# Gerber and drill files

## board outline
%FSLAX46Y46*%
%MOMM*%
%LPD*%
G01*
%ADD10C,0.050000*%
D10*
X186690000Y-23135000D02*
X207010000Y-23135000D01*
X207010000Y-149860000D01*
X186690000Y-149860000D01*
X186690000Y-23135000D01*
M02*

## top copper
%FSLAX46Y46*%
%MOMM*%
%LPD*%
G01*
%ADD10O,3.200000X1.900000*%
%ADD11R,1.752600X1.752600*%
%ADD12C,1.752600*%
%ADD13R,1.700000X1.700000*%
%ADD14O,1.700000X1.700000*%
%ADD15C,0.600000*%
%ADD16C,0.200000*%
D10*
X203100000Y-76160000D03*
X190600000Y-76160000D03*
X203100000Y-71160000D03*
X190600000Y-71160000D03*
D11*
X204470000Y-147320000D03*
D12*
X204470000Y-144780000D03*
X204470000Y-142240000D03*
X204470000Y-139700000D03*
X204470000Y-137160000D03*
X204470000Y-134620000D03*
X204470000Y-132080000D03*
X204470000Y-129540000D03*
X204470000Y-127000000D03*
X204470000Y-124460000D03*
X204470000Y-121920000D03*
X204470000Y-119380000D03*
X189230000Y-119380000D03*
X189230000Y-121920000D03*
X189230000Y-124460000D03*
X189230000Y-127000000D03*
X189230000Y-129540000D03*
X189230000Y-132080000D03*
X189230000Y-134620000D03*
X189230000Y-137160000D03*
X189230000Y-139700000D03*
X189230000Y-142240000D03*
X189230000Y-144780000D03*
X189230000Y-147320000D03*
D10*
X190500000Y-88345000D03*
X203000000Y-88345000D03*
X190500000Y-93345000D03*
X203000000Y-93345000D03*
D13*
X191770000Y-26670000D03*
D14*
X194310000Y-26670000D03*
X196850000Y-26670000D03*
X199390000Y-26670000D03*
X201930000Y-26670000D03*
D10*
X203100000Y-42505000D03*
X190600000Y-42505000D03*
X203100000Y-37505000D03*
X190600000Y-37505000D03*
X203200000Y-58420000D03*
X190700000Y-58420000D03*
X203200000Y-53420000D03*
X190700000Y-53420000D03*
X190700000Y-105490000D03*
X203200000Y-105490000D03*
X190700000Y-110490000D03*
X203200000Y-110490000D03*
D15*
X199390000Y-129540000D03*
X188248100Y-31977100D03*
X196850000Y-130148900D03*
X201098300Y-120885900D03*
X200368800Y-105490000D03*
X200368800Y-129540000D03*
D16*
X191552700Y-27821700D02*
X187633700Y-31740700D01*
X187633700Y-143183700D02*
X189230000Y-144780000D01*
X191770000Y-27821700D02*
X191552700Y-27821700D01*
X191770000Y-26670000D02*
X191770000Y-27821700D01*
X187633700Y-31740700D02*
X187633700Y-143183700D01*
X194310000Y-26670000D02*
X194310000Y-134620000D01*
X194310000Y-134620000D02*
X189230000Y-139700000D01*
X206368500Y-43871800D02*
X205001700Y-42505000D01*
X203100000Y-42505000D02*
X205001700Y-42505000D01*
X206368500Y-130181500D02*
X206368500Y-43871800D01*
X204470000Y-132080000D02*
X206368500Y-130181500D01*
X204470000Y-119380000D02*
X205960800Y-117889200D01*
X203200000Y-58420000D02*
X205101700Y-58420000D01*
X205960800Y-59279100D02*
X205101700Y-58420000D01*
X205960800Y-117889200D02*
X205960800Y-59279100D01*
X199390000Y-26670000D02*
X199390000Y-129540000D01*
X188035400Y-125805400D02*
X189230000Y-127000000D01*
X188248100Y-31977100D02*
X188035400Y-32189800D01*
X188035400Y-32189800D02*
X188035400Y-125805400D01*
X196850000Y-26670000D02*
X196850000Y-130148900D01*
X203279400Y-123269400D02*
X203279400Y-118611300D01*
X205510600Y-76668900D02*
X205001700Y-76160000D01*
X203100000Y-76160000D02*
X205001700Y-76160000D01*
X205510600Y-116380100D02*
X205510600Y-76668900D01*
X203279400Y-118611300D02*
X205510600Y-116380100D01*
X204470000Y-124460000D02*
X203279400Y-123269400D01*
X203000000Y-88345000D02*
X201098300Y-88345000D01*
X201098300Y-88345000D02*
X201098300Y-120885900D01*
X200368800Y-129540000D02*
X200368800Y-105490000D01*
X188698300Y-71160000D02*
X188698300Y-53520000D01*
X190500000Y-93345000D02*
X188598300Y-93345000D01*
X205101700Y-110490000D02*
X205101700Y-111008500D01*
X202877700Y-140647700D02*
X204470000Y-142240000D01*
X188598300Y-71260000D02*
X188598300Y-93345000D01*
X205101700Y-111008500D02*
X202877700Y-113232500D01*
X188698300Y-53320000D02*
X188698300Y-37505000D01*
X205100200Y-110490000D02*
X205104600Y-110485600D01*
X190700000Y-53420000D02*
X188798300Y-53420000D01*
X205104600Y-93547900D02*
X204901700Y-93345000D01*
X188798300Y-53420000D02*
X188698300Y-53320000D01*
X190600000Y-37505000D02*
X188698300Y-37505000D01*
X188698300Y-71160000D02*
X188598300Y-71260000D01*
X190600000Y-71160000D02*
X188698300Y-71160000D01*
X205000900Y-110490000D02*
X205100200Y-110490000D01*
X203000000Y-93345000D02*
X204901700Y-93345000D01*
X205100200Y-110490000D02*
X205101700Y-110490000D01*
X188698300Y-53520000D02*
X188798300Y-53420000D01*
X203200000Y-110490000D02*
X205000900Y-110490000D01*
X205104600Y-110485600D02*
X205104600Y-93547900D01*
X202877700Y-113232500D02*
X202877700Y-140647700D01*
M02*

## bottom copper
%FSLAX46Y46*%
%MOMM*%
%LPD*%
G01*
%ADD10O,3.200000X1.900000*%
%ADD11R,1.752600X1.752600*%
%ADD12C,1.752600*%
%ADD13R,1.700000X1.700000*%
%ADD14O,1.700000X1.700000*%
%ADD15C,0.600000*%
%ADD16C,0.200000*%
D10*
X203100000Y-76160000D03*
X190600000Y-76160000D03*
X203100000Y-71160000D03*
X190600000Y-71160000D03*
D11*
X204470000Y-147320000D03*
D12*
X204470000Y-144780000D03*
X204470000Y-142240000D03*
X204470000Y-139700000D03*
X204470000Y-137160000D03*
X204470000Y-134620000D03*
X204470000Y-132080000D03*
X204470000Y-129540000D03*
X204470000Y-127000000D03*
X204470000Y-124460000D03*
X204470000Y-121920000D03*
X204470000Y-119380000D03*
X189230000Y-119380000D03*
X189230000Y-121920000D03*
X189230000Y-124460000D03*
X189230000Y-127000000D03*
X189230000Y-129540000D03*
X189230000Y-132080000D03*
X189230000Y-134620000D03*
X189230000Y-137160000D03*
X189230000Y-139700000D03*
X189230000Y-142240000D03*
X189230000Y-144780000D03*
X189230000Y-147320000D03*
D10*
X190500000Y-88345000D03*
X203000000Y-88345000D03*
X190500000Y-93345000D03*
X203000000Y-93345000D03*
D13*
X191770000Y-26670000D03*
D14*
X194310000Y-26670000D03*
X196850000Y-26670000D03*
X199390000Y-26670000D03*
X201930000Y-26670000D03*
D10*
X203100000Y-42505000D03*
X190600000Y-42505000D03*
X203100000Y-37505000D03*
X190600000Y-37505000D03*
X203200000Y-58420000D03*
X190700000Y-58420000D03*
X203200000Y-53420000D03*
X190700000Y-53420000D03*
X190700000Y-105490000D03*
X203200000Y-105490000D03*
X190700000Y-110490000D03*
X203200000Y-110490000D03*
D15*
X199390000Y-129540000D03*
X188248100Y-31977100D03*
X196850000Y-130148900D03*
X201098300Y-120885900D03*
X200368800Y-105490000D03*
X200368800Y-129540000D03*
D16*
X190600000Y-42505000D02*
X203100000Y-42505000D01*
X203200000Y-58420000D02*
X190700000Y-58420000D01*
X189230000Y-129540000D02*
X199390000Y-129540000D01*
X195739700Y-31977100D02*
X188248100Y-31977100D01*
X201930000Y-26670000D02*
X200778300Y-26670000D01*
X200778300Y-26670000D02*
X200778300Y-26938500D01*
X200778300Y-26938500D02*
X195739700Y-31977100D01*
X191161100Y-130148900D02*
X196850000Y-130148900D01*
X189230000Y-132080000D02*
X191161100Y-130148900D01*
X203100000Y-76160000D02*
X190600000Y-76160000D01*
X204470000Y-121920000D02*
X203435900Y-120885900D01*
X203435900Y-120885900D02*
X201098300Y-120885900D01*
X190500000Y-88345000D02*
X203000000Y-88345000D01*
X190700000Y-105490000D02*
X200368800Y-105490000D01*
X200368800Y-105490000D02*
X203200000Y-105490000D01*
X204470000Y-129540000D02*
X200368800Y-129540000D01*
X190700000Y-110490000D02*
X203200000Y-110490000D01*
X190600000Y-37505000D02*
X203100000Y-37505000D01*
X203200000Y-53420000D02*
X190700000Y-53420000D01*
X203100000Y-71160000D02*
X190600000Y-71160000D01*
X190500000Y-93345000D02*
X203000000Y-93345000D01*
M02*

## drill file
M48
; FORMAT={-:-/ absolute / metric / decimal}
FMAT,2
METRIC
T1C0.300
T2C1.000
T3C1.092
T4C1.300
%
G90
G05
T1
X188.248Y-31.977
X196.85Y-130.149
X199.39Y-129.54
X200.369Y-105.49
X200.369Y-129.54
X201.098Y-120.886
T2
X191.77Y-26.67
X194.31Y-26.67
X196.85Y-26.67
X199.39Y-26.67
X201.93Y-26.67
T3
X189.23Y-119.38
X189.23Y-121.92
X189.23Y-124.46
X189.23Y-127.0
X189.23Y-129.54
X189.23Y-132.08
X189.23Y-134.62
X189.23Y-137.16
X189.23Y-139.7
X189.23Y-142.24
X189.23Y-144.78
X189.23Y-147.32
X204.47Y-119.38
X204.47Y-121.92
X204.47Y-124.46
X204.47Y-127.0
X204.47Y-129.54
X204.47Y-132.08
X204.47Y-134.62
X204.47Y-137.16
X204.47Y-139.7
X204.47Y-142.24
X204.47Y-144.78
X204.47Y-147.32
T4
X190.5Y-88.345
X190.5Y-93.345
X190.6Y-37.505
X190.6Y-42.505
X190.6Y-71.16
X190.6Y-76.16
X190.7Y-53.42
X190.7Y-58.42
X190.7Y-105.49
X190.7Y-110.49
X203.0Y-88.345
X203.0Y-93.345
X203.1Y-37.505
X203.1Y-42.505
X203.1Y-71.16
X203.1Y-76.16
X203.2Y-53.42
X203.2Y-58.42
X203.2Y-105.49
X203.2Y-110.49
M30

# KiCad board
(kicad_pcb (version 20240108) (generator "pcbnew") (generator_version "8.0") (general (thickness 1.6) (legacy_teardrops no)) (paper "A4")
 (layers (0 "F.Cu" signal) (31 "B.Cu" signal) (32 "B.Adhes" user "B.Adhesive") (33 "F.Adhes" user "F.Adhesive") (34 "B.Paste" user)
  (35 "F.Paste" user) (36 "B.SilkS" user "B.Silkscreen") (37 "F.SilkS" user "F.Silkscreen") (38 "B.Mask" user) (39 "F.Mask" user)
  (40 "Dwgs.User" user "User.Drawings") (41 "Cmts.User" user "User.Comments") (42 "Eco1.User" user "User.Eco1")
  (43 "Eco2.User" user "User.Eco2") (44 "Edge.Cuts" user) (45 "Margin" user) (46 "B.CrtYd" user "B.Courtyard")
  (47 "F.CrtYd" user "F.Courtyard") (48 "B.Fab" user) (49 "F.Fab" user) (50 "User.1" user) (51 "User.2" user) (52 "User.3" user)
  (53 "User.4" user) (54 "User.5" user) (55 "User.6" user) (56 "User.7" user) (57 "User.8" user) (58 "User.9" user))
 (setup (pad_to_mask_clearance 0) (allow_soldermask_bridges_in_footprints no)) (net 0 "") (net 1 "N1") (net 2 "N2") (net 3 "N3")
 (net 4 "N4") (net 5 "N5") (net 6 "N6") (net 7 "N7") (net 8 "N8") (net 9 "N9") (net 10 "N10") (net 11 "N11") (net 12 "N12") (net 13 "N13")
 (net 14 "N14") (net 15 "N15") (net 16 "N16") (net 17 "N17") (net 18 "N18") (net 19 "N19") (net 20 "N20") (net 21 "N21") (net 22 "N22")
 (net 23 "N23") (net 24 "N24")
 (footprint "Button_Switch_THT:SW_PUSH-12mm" (layer "F.Cu") (at 203.1 76.16 180)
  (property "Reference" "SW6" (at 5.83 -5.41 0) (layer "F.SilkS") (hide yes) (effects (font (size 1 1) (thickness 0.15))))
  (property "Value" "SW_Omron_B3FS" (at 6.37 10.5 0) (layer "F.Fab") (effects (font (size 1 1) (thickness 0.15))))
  (pad "1" thru_hole oval (at 0 0 180) (size 3.2 1.9) (drill 1.3) (layers "*.Cu" "*.Mask") (remove_unused_layers no) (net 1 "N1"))
  (pad "1" thru_hole oval (at 12.5 0 180) (size 3.2 1.9) (drill 1.3) (layers "*.Cu" "*.Mask") (remove_unused_layers no) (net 1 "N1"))
  (pad "2" thru_hole oval (at 0 5 180) (size 3.2 1.9) (drill 1.3) (layers "*.Cu" "*.Mask") (remove_unused_layers no) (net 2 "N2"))
  (pad "2" thru_hole oval (at 12.5 5 180) (size 3.2 1.9) (drill 1.3) (layers "*.Cu" "*.Mask") (remove_unused_layers no) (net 2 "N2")))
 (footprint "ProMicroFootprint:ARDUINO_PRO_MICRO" (layer "F.Cu") (at 196.85 133.35 90)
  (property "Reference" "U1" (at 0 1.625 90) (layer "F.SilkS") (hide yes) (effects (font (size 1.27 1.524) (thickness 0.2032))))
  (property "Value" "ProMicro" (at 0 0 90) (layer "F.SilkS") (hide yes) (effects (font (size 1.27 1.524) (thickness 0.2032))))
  (pad "1" thru_hole rect (at -13.97 7.62 90) (size 1.7526 1.7526) (drill 1.0922) (layers "*.Cu" "*.SilkS" "*.Mask")
   (remove_unused_layers no) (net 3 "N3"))
  (pad "2" thru_hole circle (at -11.43 7.62 90) (size 1.7526 1.7526) (drill 1.0922) (layers "*.Cu" "*.SilkS" "*.Mask")
   (remove_unused_layers no) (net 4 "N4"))
  (pad "3" thru_hole circle (at -8.89 7.62 90) (size 1.7526 1.7526) (drill 1.0922) (layers "*.Cu" "*.SilkS" "*.Mask")
   (remove_unused_layers no) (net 2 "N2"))
  (pad "4" thru_hole circle (at -6.35 7.62 90) (size 1.7526 1.7526) (drill 1.0922) (layers "*.Cu" "*.SilkS" "*.Mask")
   (remove_unused_layers no) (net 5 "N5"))
  (pad "5" thru_hole circle (at -3.81 7.62 90) (size 1.7526 1.7526) (drill 1.0922) (layers "*.Cu" "*.SilkS" "*.Mask")
   (remove_unused_layers no) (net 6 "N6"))
  (pad "6" thru_hole circle (at -1.27 7.62 90) (size 1.7526 1.7526) (drill 1.0922) (layers "*.Cu" "*.SilkS" "*.Mask")
   (remove_unused_layers no) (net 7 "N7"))
  (pad "7" thru_hole circle (at 1.27 7.62 90) (size 1.7526 1.7526) (drill 1.0922) (layers "*.Cu" "*.SilkS" "*.Mask")
   (remove_unused_layers no) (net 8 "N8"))
  (pad "8" thru_hole circle (at 3.81 7.62 90) (size 1.7526 1.7526) (drill 1.0922) (layers "*.Cu" "*.SilkS" "*.Mask")
   (remove_unused_layers no) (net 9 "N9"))
  (pad "9" thru_hole circle (at 6.35 7.62 90) (size 1.7526 1.7526) (drill 1.0922) (layers "*.Cu" "*.SilkS" "*.Mask")
   (remove_unused_layers no) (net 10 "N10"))
  (pad "10" thru_hole circle (at 8.89 7.62 90) (size 1.7526 1.7526) (drill 1.0922) (layers "*.Cu" "*.SilkS" "*.Mask")
   (remove_unused_layers no) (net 1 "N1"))
  (pad "11" thru_hole circle (at 11.43 7.62 90) (size 1.7526 1.7526) (drill 1.0922) (layers "*.Cu" "*.SilkS" "*.Mask")
   (remove_unused_layers no) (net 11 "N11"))
  (pad "12" thru_hole circle (at 13.97 7.62 90) (size 1.7526 1.7526) (drill 1.0922) (layers "*.Cu" "*.SilkS" "*.Mask")
   (remove_unused_layers no) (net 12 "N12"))
  (pad "13" thru_hole circle (at 13.97 -7.62 90) (size 1.7526 1.7526) (drill 1.0922) (layers "*.Cu" "*.SilkS" "*.Mask")
   (remove_unused_layers no) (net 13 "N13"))
  (pad "14" thru_hole circle (at 11.43 -7.62 90) (size 1.7526 1.7526) (drill 1.0922) (layers "*.Cu" "*.SilkS" "*.Mask")
   (remove_unused_layers no) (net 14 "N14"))
  (pad "15" thru_hole circle (at 8.89 -7.62 90) (size 1.7526 1.7526) (drill 1.0922) (layers "*.Cu" "*.SilkS" "*.Mask")
   (remove_unused_layers no) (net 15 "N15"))
  (pad "16" thru_hole circle (at 6.35 -7.62 90) (size 1.7526 1.7526) (drill 1.0922) (layers "*.Cu" "*.SilkS" "*.Mask")
   (remove_unused_layers no) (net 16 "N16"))
  (pad "17" thru_hole circle (at 3.81 -7.62 90) (size 1.7526 1.7526) (drill 1.0922) (layers "*.Cu" "*.SilkS" "*.Mask")
   (remove_unused_layers no) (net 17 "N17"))
  (pad "18" thru_hole circle (at 1.27 -7.62 90) (size 1.7526 1.7526) (drill 1.0922) (layers "*.Cu" "*.SilkS" "*.Mask")
   (remove_unused_layers no) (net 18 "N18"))
  (pad "19" thru_hole circle (at -1.27 -7.62 90) (size 1.7526 1.7526) (drill 1.0922) (layers "*.Cu" "*.SilkS" "*.Mask")
   (remove_unused_layers no) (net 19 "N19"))
  (pad "20" thru_hole circle (at -3.81 -7.62 90) (size 1.7526 1.7526) (drill 1.0922) (layers "*.Cu" "*.SilkS" "*.Mask")
   (remove_unused_layers no) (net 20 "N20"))
  (pad "21" thru_hole circle (at -6.35 -7.62 90) (size 1.7526 1.7526) (drill 1.0922) (layers "*.Cu" "*.SilkS" "*.Mask")
   (remove_unused_layers no) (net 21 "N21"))
  (pad "22" thru_hole circle (at -8.89 -7.62 90) (size 1.7526 1.7526) (drill 1.0922) (layers "*.Cu" "*.SilkS" "*.Mask")
   (remove_unused_layers no) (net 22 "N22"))
  (pad "23" thru_hole circle (at -11.43 -7.62 90) (size 1.7526 1.7526) (drill 1.0922) (layers "*.Cu" "*.SilkS" "*.Mask")
   (remove_unused_layers no) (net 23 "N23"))
  (pad "24" thru_hole circle (at -13.97 -7.62 90) (size 1.7526 1.7526) (drill 1.0922) (layers "*.Cu" "*.SilkS" "*.Mask")
   (remove_unused_layers no) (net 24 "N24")))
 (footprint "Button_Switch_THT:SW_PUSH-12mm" (layer "F.Cu") (at 190.5 88.345)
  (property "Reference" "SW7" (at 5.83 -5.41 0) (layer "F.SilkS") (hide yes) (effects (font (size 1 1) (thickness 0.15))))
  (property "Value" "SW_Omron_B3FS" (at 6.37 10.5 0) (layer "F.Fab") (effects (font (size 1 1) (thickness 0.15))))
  (pad "1" thru_hole oval (at 0 0) (size 3.2 1.9) (drill 1.3) (layers "*.Cu" "*.Mask") (remove_unused_layers no) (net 11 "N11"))
  (pad "1" thru_hole oval (at 12.5 0) (size 3.2 1.9) (drill 1.3) (layers "*.Cu" "*.Mask") (remove_unused_layers no) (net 11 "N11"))
  (pad "2" thru_hole oval (at 0 5) (size 3.2 1.9) (drill 1.3) (layers "*.Cu" "*.Mask") (remove_unused_layers no) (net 2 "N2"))
  (pad "2" thru_hole oval (at 12.5 5) (size 3.2 1.9) (drill 1.3) (layers "*.Cu" "*.Mask") (remove_unused_layers no) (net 2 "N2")))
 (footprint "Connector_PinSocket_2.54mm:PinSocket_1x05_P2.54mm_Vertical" (layer "F.Cu") (at 191.77 26.67 90)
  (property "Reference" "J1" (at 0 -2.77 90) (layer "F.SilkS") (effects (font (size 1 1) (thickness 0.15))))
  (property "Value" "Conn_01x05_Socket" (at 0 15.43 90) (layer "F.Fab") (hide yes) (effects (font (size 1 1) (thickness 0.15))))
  (pad "1" thru_hole rect (at 0 0 90) (size 1.7 1.7) (drill 1) (layers "*.Cu" "*.Mask") (remove_unused_layers no) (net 23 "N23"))
  (pad "2" thru_hole oval (at 0 2.54 90) (size 1.7 1.7) (drill 1) (layers "*.Cu" "*.Mask") (remove_unused_layers no) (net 21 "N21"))
  (pad "3" thru_hole oval (at 0 5.08 90) (size 1.7 1.7) (drill 1) (layers "*.Cu" "*.Mask") (remove_unused_layers no) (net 18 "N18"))
  (pad "4" thru_hole oval (at 0 7.62 90) (size 1.7 1.7) (drill 1) (layers "*.Cu" "*.Mask") (remove_unused_layers no) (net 17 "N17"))
  (pad "5" thru_hole oval (at 0 10.16 90) (size 1.7 1.7) (drill 1) (layers "*.Cu" "*.Mask") (remove_unused_layers no) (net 16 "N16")))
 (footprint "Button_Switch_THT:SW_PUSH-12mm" (layer "F.Cu") (at 203.1 42.505 180)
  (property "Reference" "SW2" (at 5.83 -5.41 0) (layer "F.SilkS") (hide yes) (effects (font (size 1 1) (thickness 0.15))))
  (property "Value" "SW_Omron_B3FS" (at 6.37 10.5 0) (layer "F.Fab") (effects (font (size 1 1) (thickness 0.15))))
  (pad "1" thru_hole oval (at 0 0 180) (size 3.2 1.9) (drill 1.3) (layers "*.Cu" "*.Mask") (remove_unused_layers no) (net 8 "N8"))
  (pad "1" thru_hole oval (at 12.5 0 180) (size 3.2 1.9) (drill 1.3) (layers "*.Cu" "*.Mask") (remove_unused_layers no) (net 8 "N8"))
  (pad "2" thru_hole oval (at 0 5 180) (size 3.2 1.9) (drill 1.3) (layers "*.Cu" "*.Mask") (remove_unused_layers no) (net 2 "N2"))
  (pad "2" thru_hole oval (at 12.5 5 180) (size 3.2 1.9) (drill 1.3) (layers "*.Cu" "*.Mask") (remove_unused_layers no) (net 2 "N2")))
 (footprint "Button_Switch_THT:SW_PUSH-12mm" (layer "F.Cu") (at 203.2 58.42 180)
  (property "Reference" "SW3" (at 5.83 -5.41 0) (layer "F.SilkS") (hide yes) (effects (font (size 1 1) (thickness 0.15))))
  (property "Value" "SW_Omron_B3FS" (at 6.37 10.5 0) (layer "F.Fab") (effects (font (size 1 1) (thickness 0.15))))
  (pad "1" thru_hole oval (at 0 0 180) (size 3.2 1.9) (drill 1.3) (layers "*.Cu" "*.Mask") (remove_unused_layers no) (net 12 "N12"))
  (pad "1" thru_hole oval (at 12.5 0 180) (size 3.2 1.9) (drill 1.3) (layers "*.Cu" "*.Mask") (remove_unused_layers no) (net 12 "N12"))
  (pad "2" thru_hole oval (at 0 5 180) (size 3.2 1.9) (drill 1.3) (layers "*.Cu" "*.Mask") (remove_unused_layers no) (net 2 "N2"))
  (pad "2" thru_hole oval (at 12.5 5 180) (size 3.2 1.9) (drill 1.3) (layers "*.Cu" "*.Mask") (remove_unused_layers no) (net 2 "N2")))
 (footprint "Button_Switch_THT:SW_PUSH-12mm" (layer "F.Cu") (at 190.7 105.49)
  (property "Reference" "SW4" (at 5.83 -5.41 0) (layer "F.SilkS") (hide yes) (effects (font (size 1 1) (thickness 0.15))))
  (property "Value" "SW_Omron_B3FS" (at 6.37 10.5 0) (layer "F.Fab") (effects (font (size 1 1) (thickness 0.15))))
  (pad "1" thru_hole oval (at 0 0) (size 3.2 1.9) (drill 1.3) (layers "*.Cu" "*.Mask") (remove_unused_layers no) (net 9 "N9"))
  (pad "1" thru_hole oval (at 12.5 0) (size 3.2 1.9) (drill 1.3) (layers "*.Cu" "*.Mask") (remove_unused_layers no) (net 9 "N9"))
  (pad "2" thru_hole oval (at 0 5) (size 3.2 1.9) (drill 1.3) (layers "*.Cu" "*.Mask") (remove_unused_layers no) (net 2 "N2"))
  (pad "2" thru_hole oval (at 12.5 5) (size 3.2 1.9) (drill 1.3) (layers "*.Cu" "*.Mask") (remove_unused_layers no) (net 2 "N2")))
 (gr_rect (start 186.69 23.135) (end 207.01 149.86) (stroke (width 0.05) (type default)) (fill none) (layer "Edge.Cuts"))
 (segment (start 191.5527 27.8217) (end 187.6337 31.7407) (width 0.2) (layer "F.Cu") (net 23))
 (segment (start 187.6337 143.1837) (end 189.23 144.78) (width 0.2) (layer "F.Cu") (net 23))
 (segment (start 191.77 27.8217) (end 191.5527 27.8217) (width 0.2) (layer "F.Cu") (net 23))
 (segment (start 191.77 26.67) (end 191.77 27.8217) (width 0.2) (layer "F.Cu") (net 23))
 (segment (start 187.6337 31.7407) (end 187.6337 143.1837) (width 0.2) (layer "F.Cu") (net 23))
 (segment (start 194.31 26.67) (end 194.31 134.62) (width 0.2) (layer "F.Cu") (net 21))
 (segment (start 194.31 134.62) (end 189.23 139.7) (width 0.2) (layer "F.Cu") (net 21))
 (segment (start 206.3685 43.8718) (end 205.0017 42.505) (width 0.2) (layer "F.Cu") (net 8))
 (segment (start 203.1 42.505) (end 205.0017 42.505) (width 0.2) (layer "F.Cu") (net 8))
 (segment (start 206.3685 130.1815) (end 206.3685 43.8718) (width 0.2) (layer "F.Cu") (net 8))
 (segment (start 204.47 132.08) (end 206.3685 130.1815) (width 0.2) (layer "F.Cu") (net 8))
 (segment (start 190.6 42.505) (end 203.1 42.505) (width 0.2) (layer "B.Cu") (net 8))
 (segment (start 204.47 119.38) (end 205.9608 117.8892) (width 0.2) (layer "F.Cu") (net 12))
 (segment (start 203.2 58.42) (end 205.1017 58.42) (width 0.2) (layer "F.Cu") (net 12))
 (segment (start 205.9608 59.2791) (end 205.1017 58.42) (width 0.2) (layer "F.Cu") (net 12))
 (segment (start 205.9608 117.8892) (end 205.9608 59.2791) (width 0.2) (layer "F.Cu") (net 12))
 (segment (start 203.2 58.42) (end 190.7 58.42) (width 0.2) (layer "B.Cu") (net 12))
 (segment (start 199.39 26.67) (end 199.39 129.54) (width 0.2) (layer "F.Cu") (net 17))
 (via (at 199.39 129.54) (size 0.6) (drill 0.3) (layers "F.Cu" "B.Cu") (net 17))
 (segment (start 189.23 129.54) (end 199.39 129.54) (width 0.2) (layer "B.Cu") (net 17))
 (segment (start 188.0354 125.8054) (end 189.23 127) (width 0.2) (layer "F.Cu") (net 16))
 (segment (start 188.2481 31.9771) (end 188.0354 32.1898) (width 0.2) (layer "F.Cu") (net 16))
 (segment (start 188.0354 32.1898) (end 188.0354 125.8054) (width 0.2) (layer "F.Cu") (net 16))
 (via (at 188.2481 31.9771) (size 0.6) (drill 0.3) (layers "F.Cu" "B.Cu") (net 16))
 (segment (start 195.7397 31.9771) (end 188.2481 31.9771) (width 0.2) (layer "B.Cu") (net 16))
 (segment (start 201.93 26.67) (end 200.7783 26.67) (width 0.2) (layer "B.Cu") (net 16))
 (segment (start 200.7783 26.67) (end 200.7783 26.9385) (width 0.2) (layer "B.Cu") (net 16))
 (segment (start 200.7783 26.9385) (end 195.7397 31.9771) (width 0.2) (layer "B.Cu") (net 16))
 (segment (start 196.85 26.67) (end 196.85 130.1489) (width 0.2) (layer "F.Cu") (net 18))
 (via (at 196.85 130.1489) (size 0.6) (drill 0.3) (layers "F.Cu" "B.Cu") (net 18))
 (segment (start 191.1611 130.1489) (end 196.85 130.1489) (width 0.2) (layer "B.Cu") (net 18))
 (segment (start 189.23 132.08) (end 191.1611 130.1489) (width 0.2) (layer "B.Cu") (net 18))
 (segment (start 203.2794 123.2694) (end 203.2794 118.6113) (width 0.2) (layer "F.Cu") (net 1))
 (segment (start 205.5106 76.6689) (end 205.0017 76.16) (width 0.2) (layer "F.Cu") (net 1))
 (segment (start 203.1 76.16) (end 205.0017 76.16) (width 0.2) (layer "F.Cu") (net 1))
 (segment (start 205.5106 116.3801) (end 205.5106 76.6689) (width 0.2) (layer "F.Cu") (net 1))
 (segment (start 203.2794 118.6113) (end 205.5106 116.3801) (width 0.2) (layer "F.Cu") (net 1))
 (segment (start 204.47 124.46) (end 203.2794 123.2694) (width 0.2) (layer "F.Cu") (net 1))
 (segment (start 203.1 76.16) (end 190.6 76.16) (width 0.2) (layer "B.Cu") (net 1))
 (segment (start 203 88.345) (end 201.0983 88.345) (width 0.2) (layer "F.Cu") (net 11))
 (segment (start 201.0983 88.345) (end 201.0983 120.8859) (width 0.2) (layer "F.Cu") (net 11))
 (via (at 201.0983 120.8859) (size 0.6) (drill 0.3) (layers "F.Cu" "B.Cu") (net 11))
 (segment (start 204.47 121.92) (end 203.4359 120.8859) (width 0.2) (layer "B.Cu") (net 11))
 (segment (start 203.4359 120.8859) (end 201.0983 120.8859) (width 0.2) (layer "B.Cu") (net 11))
 (segment (start 190.5 88.345) (end 203 88.345) (width 0.2) (layer "B.Cu") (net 11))
 (segment (start 200.3688 129.54) (end 200.3688 105.49) (width 0.2) (layer "F.Cu") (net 9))
 (via (at 200.3688 105.49) (size 0.6) (drill 0.3) (layers "F.Cu" "B.Cu") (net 9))
 (via (at 200.3688 129.54) (size 0.6) (drill 0.3) (layers "F.Cu" "B.Cu") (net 9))
 (segment (start 190.7 105.49) (end 200.3688 105.49) (width 0.2) (layer "B.Cu") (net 9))
 (segment (start 200.3688 105.49) (end 203.2 105.49) (width 0.2) (layer "B.Cu") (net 9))
 (segment (start 204.47 129.54) (end 200.3688 129.54) (width 0.2) (layer "B.Cu") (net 9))
 (segment (start 188.6983 71.16) (end 188.6983 53.52) (width 0.2) (layer "F.Cu") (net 2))
 (segment (start 190.5 93.345) (end 188.5983 93.345) (width 0.2) (layer "F.Cu") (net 2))
 (segment (start 205.1017 110.49) (end 205.1017 111.0085) (width 0.2) (layer "F.Cu") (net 2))
 (segment (start 202.8777 140.6477) (end 204.47 142.24) (width 0.2) (layer "F.Cu") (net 2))
 (segment (start 188.5983 71.26) (end 188.5983 93.345) (width 0.2) (layer "F.Cu") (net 2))
 (segment (start 205.1017 111.0085) (end 202.8777 113.2325) (width 0.2) (layer "F.Cu") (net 2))
 (segment (start 188.6983 53.32) (end 188.6983 37.505) (width 0.2) (layer "F.Cu") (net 2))
 (segment (start 205.1002 110.49) (end 205.1046 110.4856) (width 0.2) (layer "F.Cu") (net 2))
 (segment (start 190.7 53.42) (end 188.7983 53.42) (width 0.2) (layer "F.Cu") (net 2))
 (segment (start 205.1046 93.5479) (end 204.9017 93.345) (width 0.2) (layer "F.Cu") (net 2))
 (segment (start 188.7983 53.42) (end 188.6983 53.32) (width 0.2) (layer "F.Cu") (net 2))
 (segment (start 190.6 37.505) (end 188.6983 37.505) (width 0.2) (layer "F.Cu") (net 2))
 (segment (start 188.6983 71.16) (end 188.5983 71.26) (width 0.2) (layer "F.Cu") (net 2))
 (segment (start 190.6 71.16) (end 188.6983 71.16) (width 0.2) (layer "F.Cu") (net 2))
 (segment (start 205.0009 110.49) (end 205.1002 110.49) (width 0.2) (layer "F.Cu") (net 2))
 (segment (start 203 93.345) (end 204.9017 93.345) (width 0.2) (layer "F.Cu") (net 2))
 (segment (start 205.1002 110.49) (end 205.1017 110.49) (width 0.2) (layer "F.Cu") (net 2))
 (segment (start 188.6983 53.52) (end 188.7983 53.42) (width 0.2) (layer "F.Cu") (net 2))
 (segment (start 203.2 110.49) (end 205.0009 110.49) (width 0.2) (layer "F.Cu") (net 2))
 (segment (start 205.1046 110.4856) (end 205.1046 93.5479) (width 0.2) (layer "F.Cu") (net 2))
 (segment (start 202.8777 113.2325) (end 202.8777 140.6477) (width 0.2) (layer "F.Cu") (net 2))
 (segment (start 190.7 110.49) (end 203.2 110.49) (width 0.2) (layer "B.Cu") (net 2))
 (segment (start 190.6 37.505) (end 203.1 37.505) (width 0.2) (layer "B.Cu") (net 2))
 (segment (start 203.2 53.42) (end 190.7 53.42) (width 0.2) (layer "B.Cu") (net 2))
 (segment (start 203.1 71.16) (end 190.6 71.16) (width 0.2) (layer "B.Cu") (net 2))
 (segment (start 190.5 93.345) (end 203 93.345) (width 0.2) (layer "B.Cu") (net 2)))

